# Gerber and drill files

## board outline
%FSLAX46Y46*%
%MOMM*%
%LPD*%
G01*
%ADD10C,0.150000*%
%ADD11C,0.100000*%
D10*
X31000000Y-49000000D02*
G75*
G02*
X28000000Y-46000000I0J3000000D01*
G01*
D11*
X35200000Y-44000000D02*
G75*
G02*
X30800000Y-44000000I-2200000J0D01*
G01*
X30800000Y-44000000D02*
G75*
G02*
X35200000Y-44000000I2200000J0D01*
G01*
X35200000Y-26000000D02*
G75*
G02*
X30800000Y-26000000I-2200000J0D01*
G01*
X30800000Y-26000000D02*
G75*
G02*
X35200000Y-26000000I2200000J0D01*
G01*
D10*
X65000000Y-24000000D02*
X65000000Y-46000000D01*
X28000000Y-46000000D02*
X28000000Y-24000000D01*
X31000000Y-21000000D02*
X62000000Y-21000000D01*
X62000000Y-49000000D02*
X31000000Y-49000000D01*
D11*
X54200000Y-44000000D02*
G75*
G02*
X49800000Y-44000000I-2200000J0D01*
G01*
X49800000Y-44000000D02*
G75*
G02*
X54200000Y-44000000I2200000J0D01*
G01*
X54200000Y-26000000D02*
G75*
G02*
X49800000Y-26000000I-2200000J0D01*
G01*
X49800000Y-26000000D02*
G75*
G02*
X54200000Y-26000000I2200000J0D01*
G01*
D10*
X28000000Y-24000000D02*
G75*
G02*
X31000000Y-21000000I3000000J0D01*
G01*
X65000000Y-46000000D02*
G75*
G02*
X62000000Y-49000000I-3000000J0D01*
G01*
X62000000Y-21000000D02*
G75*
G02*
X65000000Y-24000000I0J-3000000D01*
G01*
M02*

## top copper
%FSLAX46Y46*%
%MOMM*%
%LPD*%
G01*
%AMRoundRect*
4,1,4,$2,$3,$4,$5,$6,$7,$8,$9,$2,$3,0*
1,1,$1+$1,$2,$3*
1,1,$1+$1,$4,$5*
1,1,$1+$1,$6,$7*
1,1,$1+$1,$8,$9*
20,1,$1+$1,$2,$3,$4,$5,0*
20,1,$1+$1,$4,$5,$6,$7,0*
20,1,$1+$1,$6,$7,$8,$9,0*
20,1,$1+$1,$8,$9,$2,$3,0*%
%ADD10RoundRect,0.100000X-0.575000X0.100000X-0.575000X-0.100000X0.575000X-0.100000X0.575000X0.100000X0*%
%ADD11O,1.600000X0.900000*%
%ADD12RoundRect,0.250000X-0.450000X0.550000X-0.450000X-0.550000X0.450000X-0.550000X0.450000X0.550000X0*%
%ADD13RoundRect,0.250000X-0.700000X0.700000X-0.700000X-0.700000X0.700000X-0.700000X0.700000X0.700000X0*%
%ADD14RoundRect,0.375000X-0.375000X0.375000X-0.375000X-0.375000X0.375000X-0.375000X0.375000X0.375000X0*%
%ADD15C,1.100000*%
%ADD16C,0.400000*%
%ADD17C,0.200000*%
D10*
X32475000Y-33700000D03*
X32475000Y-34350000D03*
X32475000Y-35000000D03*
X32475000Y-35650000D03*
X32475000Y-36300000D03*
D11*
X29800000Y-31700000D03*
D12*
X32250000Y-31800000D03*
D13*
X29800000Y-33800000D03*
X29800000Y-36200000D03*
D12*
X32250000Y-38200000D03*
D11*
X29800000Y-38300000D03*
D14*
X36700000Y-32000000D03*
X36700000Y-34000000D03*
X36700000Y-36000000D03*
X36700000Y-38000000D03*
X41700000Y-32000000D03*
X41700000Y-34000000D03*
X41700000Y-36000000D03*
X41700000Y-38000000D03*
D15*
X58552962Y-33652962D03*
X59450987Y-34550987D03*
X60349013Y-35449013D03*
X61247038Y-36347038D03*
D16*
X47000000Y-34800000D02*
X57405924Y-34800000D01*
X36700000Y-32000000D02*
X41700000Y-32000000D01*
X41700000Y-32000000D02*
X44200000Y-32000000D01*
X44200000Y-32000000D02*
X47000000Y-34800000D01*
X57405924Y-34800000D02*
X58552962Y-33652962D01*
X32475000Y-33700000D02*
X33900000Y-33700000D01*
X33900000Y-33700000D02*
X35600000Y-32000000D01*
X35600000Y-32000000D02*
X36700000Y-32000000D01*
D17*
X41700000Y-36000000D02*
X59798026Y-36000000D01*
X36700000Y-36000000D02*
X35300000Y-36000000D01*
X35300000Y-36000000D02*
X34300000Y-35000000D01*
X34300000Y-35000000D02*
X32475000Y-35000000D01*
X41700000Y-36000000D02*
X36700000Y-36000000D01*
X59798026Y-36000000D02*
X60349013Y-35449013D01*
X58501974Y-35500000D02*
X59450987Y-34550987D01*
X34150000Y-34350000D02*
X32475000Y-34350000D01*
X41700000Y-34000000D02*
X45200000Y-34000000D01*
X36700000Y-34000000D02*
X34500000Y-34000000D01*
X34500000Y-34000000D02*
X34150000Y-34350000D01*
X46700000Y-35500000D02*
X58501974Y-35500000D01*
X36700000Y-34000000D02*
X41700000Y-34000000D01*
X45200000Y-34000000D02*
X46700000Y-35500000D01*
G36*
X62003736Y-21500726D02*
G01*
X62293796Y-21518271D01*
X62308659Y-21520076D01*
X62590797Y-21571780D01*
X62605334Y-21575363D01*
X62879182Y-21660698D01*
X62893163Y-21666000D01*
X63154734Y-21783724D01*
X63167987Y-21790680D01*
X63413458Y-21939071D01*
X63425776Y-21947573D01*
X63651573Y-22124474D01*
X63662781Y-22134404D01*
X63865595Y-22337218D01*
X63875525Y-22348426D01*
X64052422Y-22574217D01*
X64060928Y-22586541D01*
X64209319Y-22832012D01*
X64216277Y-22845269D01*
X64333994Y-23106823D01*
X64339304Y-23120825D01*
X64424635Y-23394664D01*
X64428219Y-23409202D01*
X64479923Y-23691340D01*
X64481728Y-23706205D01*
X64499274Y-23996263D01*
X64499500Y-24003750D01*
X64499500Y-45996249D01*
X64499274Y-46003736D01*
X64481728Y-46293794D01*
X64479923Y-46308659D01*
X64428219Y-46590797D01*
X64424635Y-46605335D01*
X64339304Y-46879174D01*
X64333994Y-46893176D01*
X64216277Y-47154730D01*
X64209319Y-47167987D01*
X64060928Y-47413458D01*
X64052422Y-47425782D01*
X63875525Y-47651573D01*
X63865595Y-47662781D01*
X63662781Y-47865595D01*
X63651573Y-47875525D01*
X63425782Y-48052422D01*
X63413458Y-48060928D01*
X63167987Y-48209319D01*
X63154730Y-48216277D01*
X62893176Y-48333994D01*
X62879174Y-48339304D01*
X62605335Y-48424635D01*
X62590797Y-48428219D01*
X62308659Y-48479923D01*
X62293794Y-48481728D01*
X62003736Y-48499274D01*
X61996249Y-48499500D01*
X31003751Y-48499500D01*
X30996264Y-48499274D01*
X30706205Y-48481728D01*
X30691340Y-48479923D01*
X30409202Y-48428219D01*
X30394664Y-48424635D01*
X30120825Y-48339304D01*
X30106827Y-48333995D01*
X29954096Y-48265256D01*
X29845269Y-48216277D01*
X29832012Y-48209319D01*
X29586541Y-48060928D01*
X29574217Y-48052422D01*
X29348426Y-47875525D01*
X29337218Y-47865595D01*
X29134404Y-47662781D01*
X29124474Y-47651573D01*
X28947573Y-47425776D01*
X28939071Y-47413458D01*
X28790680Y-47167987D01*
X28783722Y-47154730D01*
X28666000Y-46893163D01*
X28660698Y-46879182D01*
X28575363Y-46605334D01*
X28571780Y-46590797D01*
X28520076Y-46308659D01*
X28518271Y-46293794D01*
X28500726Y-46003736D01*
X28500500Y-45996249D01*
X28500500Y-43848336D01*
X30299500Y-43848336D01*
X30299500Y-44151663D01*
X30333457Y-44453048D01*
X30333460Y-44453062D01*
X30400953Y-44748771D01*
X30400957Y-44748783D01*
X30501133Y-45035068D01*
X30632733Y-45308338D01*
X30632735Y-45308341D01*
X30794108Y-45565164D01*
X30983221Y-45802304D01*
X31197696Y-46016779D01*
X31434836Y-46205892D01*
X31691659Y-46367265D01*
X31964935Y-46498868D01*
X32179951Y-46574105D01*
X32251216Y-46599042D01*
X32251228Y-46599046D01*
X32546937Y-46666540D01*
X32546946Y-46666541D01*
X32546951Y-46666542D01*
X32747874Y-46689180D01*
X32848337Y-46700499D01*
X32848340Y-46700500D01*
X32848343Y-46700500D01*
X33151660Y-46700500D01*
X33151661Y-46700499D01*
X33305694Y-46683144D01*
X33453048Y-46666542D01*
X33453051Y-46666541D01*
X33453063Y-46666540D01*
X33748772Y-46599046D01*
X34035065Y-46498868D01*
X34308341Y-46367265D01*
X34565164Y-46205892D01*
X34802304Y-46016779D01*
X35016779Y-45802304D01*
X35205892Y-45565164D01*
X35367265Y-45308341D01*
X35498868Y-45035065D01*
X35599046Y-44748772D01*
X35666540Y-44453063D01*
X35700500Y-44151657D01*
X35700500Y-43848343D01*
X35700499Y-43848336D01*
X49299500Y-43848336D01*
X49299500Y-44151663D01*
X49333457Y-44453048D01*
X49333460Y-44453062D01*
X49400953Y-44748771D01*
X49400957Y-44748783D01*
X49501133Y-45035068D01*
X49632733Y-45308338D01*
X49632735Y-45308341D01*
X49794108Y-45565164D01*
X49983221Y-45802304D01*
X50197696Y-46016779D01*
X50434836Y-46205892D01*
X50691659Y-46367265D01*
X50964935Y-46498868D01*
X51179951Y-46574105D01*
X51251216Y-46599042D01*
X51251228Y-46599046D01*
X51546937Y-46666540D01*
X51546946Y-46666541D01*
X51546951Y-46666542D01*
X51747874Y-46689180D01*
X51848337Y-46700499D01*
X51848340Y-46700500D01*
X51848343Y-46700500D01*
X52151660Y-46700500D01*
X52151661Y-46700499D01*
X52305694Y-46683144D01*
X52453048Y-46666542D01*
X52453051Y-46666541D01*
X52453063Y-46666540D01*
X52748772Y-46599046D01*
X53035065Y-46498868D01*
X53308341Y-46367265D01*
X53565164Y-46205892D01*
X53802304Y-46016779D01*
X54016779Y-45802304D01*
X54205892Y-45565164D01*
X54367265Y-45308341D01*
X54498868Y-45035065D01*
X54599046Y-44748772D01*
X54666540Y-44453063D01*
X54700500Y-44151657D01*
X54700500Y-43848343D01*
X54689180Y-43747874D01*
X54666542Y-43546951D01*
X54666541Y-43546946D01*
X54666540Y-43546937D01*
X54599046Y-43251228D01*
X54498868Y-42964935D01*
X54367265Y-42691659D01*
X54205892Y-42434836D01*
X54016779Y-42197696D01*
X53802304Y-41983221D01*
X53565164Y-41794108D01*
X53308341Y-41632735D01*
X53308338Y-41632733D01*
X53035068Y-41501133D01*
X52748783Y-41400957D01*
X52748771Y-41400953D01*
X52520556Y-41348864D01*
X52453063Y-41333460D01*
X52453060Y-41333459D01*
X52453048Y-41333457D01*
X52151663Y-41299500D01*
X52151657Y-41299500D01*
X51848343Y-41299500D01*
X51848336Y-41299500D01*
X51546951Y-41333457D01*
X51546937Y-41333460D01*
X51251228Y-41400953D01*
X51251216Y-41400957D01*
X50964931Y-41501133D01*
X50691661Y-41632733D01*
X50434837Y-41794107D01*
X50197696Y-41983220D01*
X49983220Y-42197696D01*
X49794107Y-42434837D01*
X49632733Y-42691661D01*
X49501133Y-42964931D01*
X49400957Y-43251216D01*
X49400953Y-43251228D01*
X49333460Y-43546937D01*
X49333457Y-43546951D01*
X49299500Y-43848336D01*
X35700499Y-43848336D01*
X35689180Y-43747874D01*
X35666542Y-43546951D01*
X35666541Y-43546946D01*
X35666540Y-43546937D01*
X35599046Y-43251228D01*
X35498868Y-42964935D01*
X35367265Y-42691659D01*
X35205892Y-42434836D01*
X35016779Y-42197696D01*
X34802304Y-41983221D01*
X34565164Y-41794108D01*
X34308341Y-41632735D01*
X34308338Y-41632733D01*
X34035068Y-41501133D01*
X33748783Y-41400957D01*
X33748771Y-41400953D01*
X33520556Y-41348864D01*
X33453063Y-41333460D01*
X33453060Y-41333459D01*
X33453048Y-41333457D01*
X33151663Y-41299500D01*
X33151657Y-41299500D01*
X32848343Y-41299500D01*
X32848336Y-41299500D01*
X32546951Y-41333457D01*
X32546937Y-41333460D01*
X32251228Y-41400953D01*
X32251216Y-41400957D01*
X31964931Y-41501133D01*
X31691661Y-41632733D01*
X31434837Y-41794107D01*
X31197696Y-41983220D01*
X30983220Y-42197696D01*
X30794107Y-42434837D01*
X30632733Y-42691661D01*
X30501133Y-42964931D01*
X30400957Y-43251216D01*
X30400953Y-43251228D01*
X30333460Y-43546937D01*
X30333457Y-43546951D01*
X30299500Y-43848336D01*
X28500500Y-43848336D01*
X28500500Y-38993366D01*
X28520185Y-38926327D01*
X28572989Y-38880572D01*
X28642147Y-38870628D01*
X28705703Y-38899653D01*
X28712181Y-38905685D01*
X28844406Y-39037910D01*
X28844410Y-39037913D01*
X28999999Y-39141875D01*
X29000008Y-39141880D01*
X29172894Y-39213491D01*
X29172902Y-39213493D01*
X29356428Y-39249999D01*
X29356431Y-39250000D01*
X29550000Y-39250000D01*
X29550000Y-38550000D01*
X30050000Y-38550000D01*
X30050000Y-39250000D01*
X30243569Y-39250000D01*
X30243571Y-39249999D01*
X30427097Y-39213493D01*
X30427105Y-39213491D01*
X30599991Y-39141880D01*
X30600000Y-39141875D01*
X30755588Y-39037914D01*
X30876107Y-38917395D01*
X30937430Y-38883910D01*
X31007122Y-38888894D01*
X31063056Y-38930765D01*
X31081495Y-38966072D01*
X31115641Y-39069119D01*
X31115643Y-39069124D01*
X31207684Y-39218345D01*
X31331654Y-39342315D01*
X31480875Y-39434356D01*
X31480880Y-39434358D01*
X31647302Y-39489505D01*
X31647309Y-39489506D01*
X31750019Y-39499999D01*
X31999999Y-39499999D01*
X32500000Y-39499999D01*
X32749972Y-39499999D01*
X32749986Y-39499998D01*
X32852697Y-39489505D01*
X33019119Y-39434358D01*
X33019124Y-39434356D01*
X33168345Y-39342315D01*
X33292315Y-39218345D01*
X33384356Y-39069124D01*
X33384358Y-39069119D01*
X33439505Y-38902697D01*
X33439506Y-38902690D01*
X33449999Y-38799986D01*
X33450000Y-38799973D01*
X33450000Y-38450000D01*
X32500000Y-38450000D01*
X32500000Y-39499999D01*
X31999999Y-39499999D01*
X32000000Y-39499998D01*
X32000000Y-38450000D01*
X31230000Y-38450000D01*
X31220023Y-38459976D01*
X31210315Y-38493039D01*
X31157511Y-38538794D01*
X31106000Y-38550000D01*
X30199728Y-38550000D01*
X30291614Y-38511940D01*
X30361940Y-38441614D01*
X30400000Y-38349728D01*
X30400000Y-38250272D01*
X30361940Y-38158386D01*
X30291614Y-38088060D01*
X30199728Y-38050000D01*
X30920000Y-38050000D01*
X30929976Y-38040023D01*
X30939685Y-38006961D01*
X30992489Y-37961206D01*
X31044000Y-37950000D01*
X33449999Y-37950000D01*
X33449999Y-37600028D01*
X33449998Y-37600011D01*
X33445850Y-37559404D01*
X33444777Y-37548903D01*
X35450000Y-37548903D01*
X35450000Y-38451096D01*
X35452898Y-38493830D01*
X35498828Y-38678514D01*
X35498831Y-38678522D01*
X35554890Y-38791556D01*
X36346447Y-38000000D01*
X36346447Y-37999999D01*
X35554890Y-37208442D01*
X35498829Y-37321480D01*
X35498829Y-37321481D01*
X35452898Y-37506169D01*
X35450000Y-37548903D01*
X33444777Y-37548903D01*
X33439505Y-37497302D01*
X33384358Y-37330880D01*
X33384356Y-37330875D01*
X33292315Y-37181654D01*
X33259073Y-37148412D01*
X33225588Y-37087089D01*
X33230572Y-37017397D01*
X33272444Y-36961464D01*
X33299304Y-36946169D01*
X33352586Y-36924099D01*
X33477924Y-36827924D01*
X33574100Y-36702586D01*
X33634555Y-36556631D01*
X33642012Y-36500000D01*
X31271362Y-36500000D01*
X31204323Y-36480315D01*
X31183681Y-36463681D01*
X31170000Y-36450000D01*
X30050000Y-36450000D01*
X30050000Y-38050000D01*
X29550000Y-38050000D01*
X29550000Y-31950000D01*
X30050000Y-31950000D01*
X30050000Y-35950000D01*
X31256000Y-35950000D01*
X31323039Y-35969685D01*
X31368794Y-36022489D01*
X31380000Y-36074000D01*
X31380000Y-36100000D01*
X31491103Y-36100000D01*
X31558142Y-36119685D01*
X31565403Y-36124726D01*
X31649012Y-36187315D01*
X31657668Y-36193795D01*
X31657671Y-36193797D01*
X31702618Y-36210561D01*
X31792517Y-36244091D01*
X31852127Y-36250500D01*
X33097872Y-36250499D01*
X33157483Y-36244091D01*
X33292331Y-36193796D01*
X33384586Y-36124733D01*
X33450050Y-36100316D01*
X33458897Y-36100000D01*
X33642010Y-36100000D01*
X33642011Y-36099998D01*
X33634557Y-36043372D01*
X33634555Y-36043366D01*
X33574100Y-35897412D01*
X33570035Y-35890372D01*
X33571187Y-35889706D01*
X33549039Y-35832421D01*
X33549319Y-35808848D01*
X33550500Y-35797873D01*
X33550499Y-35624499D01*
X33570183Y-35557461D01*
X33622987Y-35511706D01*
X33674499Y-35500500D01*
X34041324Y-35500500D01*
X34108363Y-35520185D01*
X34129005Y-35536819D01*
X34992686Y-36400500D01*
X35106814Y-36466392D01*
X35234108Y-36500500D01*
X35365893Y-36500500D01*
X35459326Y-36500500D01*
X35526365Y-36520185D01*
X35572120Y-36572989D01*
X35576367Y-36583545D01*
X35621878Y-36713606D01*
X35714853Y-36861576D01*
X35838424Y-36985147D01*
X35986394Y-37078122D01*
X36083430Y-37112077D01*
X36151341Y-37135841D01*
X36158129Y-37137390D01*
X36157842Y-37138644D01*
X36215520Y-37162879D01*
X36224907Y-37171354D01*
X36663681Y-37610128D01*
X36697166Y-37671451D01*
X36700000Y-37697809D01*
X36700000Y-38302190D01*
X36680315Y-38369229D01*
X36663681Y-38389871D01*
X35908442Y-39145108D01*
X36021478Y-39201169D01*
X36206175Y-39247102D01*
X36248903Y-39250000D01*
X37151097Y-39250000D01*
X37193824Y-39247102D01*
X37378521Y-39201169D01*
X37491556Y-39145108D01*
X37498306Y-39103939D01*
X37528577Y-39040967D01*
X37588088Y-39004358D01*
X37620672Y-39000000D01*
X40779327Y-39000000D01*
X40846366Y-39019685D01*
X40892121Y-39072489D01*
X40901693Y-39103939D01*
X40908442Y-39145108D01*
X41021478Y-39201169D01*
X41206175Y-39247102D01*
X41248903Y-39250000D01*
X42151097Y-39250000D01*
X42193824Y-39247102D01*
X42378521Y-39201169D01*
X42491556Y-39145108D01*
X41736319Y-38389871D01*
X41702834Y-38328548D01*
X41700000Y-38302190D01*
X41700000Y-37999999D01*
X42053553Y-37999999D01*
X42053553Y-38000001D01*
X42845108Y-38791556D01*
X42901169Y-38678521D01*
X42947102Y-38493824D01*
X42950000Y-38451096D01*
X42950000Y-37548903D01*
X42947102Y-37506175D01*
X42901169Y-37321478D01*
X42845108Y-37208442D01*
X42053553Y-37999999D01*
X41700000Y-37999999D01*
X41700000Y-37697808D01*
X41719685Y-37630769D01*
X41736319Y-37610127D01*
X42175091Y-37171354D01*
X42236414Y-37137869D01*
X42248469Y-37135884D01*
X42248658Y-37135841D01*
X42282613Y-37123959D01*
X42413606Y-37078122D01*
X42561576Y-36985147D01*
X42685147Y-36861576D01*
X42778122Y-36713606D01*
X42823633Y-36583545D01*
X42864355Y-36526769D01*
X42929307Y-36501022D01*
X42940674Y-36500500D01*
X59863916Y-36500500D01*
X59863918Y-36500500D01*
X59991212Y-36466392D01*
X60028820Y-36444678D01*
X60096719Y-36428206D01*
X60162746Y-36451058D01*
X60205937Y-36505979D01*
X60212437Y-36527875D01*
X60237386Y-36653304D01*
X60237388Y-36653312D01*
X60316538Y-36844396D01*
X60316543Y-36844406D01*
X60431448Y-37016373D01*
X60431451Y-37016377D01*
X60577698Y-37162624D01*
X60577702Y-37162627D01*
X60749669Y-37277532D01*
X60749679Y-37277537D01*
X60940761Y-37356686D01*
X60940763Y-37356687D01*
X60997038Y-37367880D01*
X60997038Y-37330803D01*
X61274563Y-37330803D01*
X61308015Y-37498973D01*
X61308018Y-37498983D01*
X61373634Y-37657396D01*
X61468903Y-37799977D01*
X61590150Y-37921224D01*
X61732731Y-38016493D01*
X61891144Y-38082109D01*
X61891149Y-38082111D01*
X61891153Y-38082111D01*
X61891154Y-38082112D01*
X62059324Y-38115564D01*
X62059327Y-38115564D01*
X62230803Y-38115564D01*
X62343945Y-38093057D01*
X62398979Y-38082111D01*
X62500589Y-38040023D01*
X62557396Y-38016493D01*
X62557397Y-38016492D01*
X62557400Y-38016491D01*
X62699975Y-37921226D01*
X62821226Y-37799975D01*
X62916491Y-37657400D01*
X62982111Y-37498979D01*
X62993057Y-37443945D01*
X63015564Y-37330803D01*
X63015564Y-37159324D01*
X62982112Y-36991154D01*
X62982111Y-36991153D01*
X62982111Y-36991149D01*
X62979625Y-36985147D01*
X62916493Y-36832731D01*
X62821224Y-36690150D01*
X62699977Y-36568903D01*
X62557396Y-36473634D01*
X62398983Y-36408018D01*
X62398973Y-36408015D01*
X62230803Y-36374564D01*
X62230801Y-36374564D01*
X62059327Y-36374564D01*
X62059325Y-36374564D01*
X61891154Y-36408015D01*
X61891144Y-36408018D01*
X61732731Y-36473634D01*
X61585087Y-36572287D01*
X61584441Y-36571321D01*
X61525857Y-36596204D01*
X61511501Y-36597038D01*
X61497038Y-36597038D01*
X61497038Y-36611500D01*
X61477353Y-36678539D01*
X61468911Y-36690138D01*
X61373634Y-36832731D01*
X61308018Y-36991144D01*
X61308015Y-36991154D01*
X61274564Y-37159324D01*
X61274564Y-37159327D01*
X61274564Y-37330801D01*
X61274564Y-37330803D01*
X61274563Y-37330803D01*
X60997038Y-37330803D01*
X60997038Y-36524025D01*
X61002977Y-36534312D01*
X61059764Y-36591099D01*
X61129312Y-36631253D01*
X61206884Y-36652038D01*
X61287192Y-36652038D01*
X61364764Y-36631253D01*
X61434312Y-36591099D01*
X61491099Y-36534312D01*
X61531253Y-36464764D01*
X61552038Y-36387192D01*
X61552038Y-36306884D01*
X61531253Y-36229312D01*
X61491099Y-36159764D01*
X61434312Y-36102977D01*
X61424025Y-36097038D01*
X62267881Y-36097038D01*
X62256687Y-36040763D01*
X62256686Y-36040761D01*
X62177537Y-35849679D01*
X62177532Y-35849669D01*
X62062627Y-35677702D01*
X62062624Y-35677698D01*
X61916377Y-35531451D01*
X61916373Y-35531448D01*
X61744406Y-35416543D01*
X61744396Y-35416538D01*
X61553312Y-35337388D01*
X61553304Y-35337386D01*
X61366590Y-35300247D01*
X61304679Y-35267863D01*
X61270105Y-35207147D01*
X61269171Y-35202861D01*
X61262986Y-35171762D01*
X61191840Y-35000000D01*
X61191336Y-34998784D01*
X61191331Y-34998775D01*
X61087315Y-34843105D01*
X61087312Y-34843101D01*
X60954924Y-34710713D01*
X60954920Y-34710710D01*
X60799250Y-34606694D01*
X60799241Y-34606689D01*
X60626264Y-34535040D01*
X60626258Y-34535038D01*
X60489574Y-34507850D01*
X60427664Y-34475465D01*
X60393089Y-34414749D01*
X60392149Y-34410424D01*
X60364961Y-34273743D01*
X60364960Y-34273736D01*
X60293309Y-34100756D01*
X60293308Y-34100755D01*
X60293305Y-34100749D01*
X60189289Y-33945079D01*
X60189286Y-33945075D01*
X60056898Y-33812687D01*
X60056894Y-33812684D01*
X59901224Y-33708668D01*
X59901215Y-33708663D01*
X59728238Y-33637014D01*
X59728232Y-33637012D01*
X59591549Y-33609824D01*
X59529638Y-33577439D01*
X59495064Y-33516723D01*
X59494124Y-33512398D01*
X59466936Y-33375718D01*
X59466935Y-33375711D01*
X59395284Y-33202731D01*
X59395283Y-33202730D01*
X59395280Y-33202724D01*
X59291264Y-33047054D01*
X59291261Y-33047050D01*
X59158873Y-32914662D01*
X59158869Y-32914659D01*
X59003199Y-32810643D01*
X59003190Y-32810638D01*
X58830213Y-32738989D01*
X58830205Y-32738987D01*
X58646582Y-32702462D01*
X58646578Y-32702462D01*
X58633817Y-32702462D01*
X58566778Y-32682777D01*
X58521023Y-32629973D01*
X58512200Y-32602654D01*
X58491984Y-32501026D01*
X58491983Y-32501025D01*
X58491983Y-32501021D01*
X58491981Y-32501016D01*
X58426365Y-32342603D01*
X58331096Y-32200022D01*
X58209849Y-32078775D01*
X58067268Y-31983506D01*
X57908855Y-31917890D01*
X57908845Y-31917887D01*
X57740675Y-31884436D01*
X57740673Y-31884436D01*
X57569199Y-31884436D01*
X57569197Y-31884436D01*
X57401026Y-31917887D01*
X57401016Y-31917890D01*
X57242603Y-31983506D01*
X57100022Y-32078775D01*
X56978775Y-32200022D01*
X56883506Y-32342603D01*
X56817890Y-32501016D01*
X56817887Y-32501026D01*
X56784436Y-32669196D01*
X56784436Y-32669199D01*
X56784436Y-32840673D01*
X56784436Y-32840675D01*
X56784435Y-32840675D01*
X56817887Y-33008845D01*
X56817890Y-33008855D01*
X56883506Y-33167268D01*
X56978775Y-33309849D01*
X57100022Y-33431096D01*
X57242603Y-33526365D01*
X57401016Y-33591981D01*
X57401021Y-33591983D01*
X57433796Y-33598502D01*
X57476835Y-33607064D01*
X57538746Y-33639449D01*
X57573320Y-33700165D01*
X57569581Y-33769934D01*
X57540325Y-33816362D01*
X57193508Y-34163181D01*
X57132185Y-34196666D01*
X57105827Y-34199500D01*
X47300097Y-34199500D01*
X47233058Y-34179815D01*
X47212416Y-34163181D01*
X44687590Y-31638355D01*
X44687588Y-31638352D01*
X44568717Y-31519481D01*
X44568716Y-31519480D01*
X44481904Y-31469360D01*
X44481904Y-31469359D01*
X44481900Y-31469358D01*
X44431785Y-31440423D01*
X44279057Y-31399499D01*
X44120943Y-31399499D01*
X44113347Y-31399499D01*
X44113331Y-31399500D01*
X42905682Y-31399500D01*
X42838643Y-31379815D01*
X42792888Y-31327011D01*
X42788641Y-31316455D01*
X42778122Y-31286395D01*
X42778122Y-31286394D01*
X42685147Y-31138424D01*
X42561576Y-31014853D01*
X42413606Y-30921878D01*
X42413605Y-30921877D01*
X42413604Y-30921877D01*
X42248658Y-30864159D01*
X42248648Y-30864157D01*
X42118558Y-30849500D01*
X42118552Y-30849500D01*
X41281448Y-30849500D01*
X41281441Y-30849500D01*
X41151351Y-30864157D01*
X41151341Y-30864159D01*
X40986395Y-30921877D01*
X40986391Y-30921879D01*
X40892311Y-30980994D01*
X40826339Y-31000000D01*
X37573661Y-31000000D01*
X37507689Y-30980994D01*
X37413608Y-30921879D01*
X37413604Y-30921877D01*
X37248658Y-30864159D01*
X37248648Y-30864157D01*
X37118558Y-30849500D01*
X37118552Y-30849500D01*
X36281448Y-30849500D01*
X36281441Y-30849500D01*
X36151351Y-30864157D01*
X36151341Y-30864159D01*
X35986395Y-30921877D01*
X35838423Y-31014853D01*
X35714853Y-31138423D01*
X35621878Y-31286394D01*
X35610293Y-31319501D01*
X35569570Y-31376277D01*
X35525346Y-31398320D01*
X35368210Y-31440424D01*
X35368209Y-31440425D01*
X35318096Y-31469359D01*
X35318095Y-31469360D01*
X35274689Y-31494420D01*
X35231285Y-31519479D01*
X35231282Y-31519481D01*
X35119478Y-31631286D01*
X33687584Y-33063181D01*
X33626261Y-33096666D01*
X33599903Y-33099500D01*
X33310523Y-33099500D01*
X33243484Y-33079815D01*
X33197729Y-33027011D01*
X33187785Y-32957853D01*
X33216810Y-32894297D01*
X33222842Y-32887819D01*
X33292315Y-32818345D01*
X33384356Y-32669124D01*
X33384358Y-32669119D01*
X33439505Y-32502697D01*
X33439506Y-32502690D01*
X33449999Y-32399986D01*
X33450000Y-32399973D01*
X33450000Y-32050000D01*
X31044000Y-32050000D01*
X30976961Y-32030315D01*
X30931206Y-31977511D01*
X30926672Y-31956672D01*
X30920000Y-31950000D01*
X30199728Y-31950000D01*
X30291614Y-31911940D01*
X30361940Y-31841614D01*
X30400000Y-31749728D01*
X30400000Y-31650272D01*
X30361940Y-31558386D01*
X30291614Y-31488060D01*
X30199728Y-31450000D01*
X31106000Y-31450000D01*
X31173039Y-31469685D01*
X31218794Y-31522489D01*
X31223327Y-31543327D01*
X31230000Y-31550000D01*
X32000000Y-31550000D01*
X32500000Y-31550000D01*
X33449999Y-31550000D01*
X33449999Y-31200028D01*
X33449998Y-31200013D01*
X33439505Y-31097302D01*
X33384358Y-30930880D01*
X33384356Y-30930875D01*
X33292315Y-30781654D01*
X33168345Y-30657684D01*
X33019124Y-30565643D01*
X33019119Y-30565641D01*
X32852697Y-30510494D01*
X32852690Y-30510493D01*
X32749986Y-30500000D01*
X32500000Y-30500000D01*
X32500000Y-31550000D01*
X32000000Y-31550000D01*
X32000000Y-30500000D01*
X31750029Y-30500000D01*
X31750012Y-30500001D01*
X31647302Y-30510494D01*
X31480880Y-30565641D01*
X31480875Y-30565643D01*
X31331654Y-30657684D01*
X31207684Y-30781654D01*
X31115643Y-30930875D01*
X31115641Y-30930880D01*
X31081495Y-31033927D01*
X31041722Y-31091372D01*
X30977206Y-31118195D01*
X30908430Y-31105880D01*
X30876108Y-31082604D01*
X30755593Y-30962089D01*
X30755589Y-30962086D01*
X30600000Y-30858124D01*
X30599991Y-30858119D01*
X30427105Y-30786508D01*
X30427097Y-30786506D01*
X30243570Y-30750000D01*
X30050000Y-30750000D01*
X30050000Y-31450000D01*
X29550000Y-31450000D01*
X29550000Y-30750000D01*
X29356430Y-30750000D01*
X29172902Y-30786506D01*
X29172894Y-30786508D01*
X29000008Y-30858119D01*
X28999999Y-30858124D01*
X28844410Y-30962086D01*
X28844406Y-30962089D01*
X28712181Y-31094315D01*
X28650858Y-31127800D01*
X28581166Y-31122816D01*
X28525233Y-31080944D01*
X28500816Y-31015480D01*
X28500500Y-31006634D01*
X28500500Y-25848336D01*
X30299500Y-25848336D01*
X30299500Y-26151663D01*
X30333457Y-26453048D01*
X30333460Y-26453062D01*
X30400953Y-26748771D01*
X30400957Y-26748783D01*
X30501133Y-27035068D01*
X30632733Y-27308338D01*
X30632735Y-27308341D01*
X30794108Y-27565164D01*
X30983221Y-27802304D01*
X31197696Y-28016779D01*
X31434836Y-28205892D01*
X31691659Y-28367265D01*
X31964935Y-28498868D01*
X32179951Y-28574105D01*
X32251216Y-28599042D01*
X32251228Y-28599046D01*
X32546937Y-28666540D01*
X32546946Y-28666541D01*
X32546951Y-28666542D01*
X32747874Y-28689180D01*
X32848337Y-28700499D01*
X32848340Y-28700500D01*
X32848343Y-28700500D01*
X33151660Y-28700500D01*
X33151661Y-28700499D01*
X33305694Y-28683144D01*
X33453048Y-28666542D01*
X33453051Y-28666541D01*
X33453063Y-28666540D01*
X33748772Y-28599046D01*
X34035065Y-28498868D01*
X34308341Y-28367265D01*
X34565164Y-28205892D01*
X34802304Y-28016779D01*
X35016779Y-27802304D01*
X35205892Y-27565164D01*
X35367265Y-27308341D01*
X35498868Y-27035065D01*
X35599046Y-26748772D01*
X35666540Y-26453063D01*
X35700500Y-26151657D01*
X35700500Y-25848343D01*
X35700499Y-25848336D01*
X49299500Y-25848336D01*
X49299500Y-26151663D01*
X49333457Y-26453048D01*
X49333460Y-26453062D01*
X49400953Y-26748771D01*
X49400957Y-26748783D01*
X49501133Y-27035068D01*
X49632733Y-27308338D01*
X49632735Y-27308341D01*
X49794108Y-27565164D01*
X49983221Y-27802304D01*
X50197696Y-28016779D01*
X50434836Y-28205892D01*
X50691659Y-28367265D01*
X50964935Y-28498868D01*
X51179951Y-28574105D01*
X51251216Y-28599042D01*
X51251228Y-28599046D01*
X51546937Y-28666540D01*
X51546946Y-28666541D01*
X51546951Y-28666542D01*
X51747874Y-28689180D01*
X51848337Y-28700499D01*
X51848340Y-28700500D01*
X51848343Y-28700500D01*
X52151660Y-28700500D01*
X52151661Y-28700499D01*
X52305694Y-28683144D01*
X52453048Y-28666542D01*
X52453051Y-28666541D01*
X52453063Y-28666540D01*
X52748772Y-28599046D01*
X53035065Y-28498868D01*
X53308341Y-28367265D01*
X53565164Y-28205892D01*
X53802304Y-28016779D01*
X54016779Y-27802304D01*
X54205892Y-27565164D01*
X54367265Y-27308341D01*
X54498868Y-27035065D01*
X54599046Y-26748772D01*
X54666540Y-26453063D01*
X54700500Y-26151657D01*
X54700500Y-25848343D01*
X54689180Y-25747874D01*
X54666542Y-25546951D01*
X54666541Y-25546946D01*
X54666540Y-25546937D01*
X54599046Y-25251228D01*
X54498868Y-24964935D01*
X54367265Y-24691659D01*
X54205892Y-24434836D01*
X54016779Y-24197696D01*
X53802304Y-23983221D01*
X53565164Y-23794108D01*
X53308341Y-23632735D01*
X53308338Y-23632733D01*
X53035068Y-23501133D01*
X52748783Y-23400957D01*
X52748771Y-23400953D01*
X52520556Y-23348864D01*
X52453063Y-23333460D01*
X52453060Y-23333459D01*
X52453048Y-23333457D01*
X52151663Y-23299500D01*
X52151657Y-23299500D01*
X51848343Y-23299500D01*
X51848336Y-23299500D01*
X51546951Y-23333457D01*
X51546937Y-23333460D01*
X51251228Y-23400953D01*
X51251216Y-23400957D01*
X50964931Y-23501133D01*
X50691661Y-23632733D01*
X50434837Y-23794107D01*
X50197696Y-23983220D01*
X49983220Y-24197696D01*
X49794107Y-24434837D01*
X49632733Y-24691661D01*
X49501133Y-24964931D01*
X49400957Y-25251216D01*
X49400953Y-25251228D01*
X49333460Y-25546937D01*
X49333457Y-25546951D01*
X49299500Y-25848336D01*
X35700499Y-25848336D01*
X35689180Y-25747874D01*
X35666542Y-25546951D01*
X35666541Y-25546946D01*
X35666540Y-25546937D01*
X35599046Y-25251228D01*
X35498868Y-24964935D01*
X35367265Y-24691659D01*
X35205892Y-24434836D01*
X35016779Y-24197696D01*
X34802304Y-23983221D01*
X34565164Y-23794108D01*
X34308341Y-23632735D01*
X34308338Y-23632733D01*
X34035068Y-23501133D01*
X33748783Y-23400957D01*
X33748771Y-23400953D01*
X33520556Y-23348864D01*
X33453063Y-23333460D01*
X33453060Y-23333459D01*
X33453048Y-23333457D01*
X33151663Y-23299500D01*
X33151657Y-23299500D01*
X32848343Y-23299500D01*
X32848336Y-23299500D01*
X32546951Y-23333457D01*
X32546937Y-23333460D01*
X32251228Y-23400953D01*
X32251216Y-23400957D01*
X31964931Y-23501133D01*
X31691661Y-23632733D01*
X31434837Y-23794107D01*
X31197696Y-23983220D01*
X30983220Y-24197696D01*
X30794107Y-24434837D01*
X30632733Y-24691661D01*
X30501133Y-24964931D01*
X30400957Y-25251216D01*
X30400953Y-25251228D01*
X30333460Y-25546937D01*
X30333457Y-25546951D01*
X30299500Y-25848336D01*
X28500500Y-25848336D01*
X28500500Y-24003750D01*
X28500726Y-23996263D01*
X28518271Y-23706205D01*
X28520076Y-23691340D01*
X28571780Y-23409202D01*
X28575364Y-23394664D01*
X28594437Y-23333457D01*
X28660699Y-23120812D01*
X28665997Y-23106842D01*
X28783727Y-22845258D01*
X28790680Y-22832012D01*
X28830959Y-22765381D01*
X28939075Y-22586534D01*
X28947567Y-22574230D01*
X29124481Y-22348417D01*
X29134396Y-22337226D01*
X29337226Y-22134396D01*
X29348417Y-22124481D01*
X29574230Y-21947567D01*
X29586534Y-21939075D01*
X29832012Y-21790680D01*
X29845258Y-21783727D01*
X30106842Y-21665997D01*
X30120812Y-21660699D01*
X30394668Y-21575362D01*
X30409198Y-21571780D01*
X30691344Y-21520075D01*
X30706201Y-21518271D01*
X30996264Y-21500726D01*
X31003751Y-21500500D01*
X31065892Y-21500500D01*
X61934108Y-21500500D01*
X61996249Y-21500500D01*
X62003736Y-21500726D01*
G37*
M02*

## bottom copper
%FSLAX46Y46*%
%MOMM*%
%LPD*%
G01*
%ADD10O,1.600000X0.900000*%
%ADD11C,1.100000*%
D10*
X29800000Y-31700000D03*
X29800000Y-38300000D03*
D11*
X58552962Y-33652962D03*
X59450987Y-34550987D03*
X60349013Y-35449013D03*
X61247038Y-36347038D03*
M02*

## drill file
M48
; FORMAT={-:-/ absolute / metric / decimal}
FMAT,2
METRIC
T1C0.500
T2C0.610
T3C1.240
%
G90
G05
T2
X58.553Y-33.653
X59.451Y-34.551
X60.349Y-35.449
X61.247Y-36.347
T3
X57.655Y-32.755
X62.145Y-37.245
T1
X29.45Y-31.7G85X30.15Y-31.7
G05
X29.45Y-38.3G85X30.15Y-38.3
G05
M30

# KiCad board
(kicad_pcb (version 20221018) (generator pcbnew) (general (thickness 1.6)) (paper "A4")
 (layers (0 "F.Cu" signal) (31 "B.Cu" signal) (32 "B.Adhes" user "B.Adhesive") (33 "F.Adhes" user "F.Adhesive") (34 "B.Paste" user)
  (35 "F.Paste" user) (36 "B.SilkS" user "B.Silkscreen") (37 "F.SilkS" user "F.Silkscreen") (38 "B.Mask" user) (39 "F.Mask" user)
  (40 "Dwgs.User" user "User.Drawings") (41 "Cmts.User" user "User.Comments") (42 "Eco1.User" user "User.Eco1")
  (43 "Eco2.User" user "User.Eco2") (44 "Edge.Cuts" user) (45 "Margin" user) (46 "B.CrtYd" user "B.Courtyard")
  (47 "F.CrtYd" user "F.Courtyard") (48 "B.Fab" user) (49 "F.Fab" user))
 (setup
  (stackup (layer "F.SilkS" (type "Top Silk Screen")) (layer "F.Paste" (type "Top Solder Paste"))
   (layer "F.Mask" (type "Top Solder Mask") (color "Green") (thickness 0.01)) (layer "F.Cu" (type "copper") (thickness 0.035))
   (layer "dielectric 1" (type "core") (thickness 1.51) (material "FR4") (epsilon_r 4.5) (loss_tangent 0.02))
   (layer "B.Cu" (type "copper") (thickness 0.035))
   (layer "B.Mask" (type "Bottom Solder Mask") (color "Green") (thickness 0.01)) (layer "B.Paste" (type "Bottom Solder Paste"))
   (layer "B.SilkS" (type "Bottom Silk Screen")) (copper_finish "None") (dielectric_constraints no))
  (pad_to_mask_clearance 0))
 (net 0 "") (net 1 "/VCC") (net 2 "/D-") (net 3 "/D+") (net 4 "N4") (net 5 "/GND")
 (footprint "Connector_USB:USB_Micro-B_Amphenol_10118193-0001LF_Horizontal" (layer "F.Cu") (at 29.8 35 -90)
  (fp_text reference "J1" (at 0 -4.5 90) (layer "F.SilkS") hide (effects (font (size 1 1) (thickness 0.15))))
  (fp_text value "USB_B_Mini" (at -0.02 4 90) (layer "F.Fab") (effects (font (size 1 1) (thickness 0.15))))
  (pad "1" smd roundrect (at -1.3 -2.675 270) (size 0.4 1.35) (layers "F.Cu" "F.Paste" "F.Mask") (roundrect_rratio 0.25) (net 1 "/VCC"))
  (pad "2" smd roundrect (at -0.65 -2.675 270) (size 0.4 1.35) (layers "F.Cu" "F.Paste" "F.Mask") (roundrect_rratio 0.25) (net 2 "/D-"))
  (pad "3" smd roundrect (at 0 -2.675 270) (size 0.4 1.35) (layers "F.Cu" "F.Paste" "F.Mask") (roundrect_rratio 0.25) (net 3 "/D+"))
  (pad "4" smd roundrect (at 0.65 -2.675 270) (size 0.4 1.35) (layers "F.Cu" "F.Paste" "F.Mask") (roundrect_rratio 0.25) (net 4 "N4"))
  (pad "5" smd roundrect (at 1.3 -2.675 270) (size 0.4 1.35) (layers "F.Cu" "F.Paste" "F.Mask") (roundrect_rratio 0.25) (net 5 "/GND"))
  (pad "6" thru_hole oval (at -3.3 0) (size 1.6 0.9) (drill oval 1.2 0.5) (layers "*.Cu" "*.Mask" "F.Paste") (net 5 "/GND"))
  (pad "6" smd roundrect (at -3.2 -2.45 270) (size 1.6 1.4) (layers "F.Cu" "F.Paste" "F.Mask") (roundrect_rratio 0.1785714286)
   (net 5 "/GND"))
  (pad "6" smd roundrect (at -1.2 0 270) (size 1.9 1.9) (layers "F.Cu" "F.Paste" "F.Mask") (roundrect_rratio 0.1315789474) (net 5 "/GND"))
  (pad "6" smd roundrect (at 1.2 0 270) (size 1.9 1.9) (layers "F.Cu" "F.Paste" "F.Mask") (roundrect_rratio 0.1315789474) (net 5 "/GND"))
  (pad "6" smd roundrect (at 3.2 -2.45 270) (size 1.6 1.4) (layers "F.Cu" "F.Paste" "F.Mask") (roundrect_rratio 0.1785714286) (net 5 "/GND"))
  (pad "6" thru_hole oval (at 3.3 0) (size 1.6 0.9) (drill oval 1.2 0.5) (layers "*.Cu" "*.Mask" "F.Paste") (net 5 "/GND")))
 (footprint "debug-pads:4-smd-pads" (layer "F.Cu") (at 36.7 35 -90)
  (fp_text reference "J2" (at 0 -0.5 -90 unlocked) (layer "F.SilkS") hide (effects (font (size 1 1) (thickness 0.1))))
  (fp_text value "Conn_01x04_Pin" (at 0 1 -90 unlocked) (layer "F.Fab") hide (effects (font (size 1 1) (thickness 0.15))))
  (pad "1" smd roundrect (at -3 0 270) (size 1.5 1.5) (layers "F.Cu" "F.Paste" "F.Mask") (roundrect_rratio 0.25) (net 1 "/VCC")
   (thermal_bridge_angle 45))
  (pad "2" smd roundrect (at -1 0 270) (size 1.5 1.5) (layers "F.Cu" "F.Paste" "F.Mask") (roundrect_rratio 0.25) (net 2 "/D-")
   (thermal_bridge_angle 45))
  (pad "3" smd roundrect (at 1 0 270) (size 1.5 1.5) (layers "F.Cu" "F.Paste" "F.Mask") (roundrect_rratio 0.25) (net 3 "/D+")
   (thermal_bridge_angle 45))
  (pad "4" smd roundrect (at 3 0 270) (size 1.5 1.5) (layers "F.Cu" "F.Paste" "F.Mask") (roundrect_rratio 0.25) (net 5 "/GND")
   (thermal_bridge_angle 45)))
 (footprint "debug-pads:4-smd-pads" (layer "F.Cu") (at 41.7 35 -90)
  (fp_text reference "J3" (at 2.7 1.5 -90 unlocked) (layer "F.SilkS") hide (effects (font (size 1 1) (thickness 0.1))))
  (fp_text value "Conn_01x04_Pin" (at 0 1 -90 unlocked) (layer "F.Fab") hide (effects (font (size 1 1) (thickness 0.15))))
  (pad "1" smd roundrect (at -3 0 270) (size 1.5 1.5) (layers "F.Cu" "F.Paste" "F.Mask") (roundrect_rratio 0.25) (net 1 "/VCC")
   (thermal_bridge_angle 45))
  (pad "2" smd roundrect (at -1 0 270) (size 1.5 1.5) (layers "F.Cu" "F.Paste" "F.Mask") (roundrect_rratio 0.25) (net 2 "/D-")
   (thermal_bridge_angle 45))
  (pad "3" smd roundrect (at 1 0 270) (size 1.5 1.5) (layers "F.Cu" "F.Paste" "F.Mask") (roundrect_rratio 0.25) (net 3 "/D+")
   (thermal_bridge_angle 45))
  (pad "4" smd roundrect (at 3 0 270) (size 1.5 1.5) (layers "F.Cu" "F.Paste" "F.Mask") (roundrect_rratio 0.25) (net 5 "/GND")
   (thermal_bridge_angle 45)))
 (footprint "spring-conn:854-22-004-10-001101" (layer "F.Cu") (at 59.9 35 -45)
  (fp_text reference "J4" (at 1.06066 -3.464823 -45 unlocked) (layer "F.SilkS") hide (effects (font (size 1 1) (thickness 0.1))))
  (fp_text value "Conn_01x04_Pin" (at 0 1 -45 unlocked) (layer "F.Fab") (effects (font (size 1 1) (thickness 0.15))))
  (pad "" np_thru_hole circle (at -3.175 0 315) (size 1.24 1.24) (drill 1.24) (layers "*.Cu" "*.Mask"))
  (pad "" np_thru_hole circle (at 3.175 0 315) (size 1.24 1.24) (drill 1.24) (layers "*.Cu" "*.Mask"))
  (pad "1" thru_hole circle (at -1.905 0 315) (size 1.1 1.1) (drill 0.61) (layers "*.Cu" "*.Mask") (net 1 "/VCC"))
  (pad "2" thru_hole circle (at -0.635 0 315) (size 1.1 1.1) (drill 0.61) (layers "*.Cu" "*.Mask") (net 2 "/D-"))
  (pad "3" thru_hole circle (at 0.635 0 315) (size 1.1 1.1) (drill 0.61) (layers "*.Cu" "*.Mask") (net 3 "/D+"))
  (pad "4" thru_hole circle (at 1.905 0 315) (size 1.1 1.1) (drill 0.61) (layers "*.Cu" "*.Mask") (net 5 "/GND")))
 (gr_arc (start 31 49) (mid 28.87868 48.12132) (end 28 46) (stroke (width 0.15) (type default)) (layer "Edge.Cuts"))
 (gr_circle (center 33 44) (end 35.2 44) (stroke (width 0.1) (type default)) (fill none) (layer "Edge.Cuts"))
 (gr_circle (center 33 26) (end 35.2 26) (stroke (width 0.1) (type default)) (fill none) (layer "Edge.Cuts"))
 (gr_line (start 65 24) (end 65 46) (stroke (width 0.15) (type default)) (layer "Edge.Cuts"))
 (gr_line (start 28 46) (end 28 24) (stroke (width 0.15) (type default)) (layer "Edge.Cuts"))
 (gr_line (start 31 21) (end 62 21) (stroke (width 0.15) (type default)) (layer "Edge.Cuts"))
 (gr_line (start 62 49) (end 31 49) (stroke (width 0.15) (type default)) (layer "Edge.Cuts"))
 (gr_circle (center 52 44) (end 54.2 44) (stroke (width 0.1) (type default)) (fill none) (layer "Edge.Cuts"))
 (gr_circle (center 52 26) (end 54.2 26) (stroke (width 0.1) (type default)) (fill none) (layer "Edge.Cuts"))
 (gr_arc (start 28 24) (mid 28.87868 21.87868) (end 31 21) (stroke (width 0.15) (type default)) (layer "Edge.Cuts"))
 (gr_arc (start 65 46) (mid 64.12132 48.12132) (end 62 49) (stroke (width 0.15) (type default)) (layer "Edge.Cuts"))
 (gr_arc (start 62 21) (mid 64.12132 21.87868) (end 65 24) (stroke (width 0.15) (type default)) (layer "Edge.Cuts"))
 (segment (start 47 34.8) (end 57.405924 34.8) (width 0.4) (layer "F.Cu") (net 1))
 (segment (start 36.7 32) (end 41.7 32) (width 0.4) (layer "F.Cu") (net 1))
 (segment (start 41.7 32) (end 44.2 32) (width 0.4) (layer "F.Cu") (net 1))
 (segment (start 44.2 32) (end 47 34.8) (width 0.4) (layer "F.Cu") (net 1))
 (segment (start 57.405924 34.8) (end 58.552962 33.652962) (width 0.4) (layer "F.Cu") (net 1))
 (segment (start 32.475 33.7) (end 33.9 33.7) (width 0.4) (layer "F.Cu") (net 1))
 (segment (start 33.9 33.7) (end 35.6 32) (width 0.4) (layer "F.Cu") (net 1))
 (segment (start 35.6 32) (end 36.7 32) (width 0.4) (layer "F.Cu") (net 1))
 (segment (start 41.7 36) (end 59.798026 36) (width 0.2) (layer "F.Cu") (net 3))
 (segment (start 36.7 36) (end 35.3 36) (width 0.2) (layer "F.Cu") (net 3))
 (segment (start 35.3 36) (end 34.3 35) (width 0.2) (layer "F.Cu") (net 3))
 (segment (start 34.3 35) (end 32.475 35) (width 0.2) (layer "F.Cu") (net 3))
 (segment (start 41.7 36) (end 36.7 36) (width 0.2) (layer "F.Cu") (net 3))
 (segment (start 59.798026 36) (end 60.349013 35.449013) (width 0.2) (layer "F.Cu") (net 3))
 (segment (start 58.501974 35.5) (end 59.450987 34.550987) (width 0.2) (layer "F.Cu") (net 2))
 (segment (start 34.15 34.35) (end 32.475 34.35) (width 0.2) (layer "F.Cu") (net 2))
 (segment (start 41.7 34) (end 45.2 34) (width 0.2) (layer "F.Cu") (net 2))
 (segment (start 36.7 34) (end 34.5 34) (width 0.2) (layer "F.Cu") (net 2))
 (segment (start 34.5 34) (end 34.15 34.35) (width 0.2) (layer "F.Cu") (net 2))
 (segment (start 46.7 35.5) (end 58.501974 35.5) (width 0.2) (layer "F.Cu") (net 2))
 (segment (start 36.7 34) (end 41.7 34) (width 0.2) (layer "F.Cu") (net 2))
 (segment (start 45.2 34) (end 46.7 35.5) (width 0.2) (layer "F.Cu") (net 2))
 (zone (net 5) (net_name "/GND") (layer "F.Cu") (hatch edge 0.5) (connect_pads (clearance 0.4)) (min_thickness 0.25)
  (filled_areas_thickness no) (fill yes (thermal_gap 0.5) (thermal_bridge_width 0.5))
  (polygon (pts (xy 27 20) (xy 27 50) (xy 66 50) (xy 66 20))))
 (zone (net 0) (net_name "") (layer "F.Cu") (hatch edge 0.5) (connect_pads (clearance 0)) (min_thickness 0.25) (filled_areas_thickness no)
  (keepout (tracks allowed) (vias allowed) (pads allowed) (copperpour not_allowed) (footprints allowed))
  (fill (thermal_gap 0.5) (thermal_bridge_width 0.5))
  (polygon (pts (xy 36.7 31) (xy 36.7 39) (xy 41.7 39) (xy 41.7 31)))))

